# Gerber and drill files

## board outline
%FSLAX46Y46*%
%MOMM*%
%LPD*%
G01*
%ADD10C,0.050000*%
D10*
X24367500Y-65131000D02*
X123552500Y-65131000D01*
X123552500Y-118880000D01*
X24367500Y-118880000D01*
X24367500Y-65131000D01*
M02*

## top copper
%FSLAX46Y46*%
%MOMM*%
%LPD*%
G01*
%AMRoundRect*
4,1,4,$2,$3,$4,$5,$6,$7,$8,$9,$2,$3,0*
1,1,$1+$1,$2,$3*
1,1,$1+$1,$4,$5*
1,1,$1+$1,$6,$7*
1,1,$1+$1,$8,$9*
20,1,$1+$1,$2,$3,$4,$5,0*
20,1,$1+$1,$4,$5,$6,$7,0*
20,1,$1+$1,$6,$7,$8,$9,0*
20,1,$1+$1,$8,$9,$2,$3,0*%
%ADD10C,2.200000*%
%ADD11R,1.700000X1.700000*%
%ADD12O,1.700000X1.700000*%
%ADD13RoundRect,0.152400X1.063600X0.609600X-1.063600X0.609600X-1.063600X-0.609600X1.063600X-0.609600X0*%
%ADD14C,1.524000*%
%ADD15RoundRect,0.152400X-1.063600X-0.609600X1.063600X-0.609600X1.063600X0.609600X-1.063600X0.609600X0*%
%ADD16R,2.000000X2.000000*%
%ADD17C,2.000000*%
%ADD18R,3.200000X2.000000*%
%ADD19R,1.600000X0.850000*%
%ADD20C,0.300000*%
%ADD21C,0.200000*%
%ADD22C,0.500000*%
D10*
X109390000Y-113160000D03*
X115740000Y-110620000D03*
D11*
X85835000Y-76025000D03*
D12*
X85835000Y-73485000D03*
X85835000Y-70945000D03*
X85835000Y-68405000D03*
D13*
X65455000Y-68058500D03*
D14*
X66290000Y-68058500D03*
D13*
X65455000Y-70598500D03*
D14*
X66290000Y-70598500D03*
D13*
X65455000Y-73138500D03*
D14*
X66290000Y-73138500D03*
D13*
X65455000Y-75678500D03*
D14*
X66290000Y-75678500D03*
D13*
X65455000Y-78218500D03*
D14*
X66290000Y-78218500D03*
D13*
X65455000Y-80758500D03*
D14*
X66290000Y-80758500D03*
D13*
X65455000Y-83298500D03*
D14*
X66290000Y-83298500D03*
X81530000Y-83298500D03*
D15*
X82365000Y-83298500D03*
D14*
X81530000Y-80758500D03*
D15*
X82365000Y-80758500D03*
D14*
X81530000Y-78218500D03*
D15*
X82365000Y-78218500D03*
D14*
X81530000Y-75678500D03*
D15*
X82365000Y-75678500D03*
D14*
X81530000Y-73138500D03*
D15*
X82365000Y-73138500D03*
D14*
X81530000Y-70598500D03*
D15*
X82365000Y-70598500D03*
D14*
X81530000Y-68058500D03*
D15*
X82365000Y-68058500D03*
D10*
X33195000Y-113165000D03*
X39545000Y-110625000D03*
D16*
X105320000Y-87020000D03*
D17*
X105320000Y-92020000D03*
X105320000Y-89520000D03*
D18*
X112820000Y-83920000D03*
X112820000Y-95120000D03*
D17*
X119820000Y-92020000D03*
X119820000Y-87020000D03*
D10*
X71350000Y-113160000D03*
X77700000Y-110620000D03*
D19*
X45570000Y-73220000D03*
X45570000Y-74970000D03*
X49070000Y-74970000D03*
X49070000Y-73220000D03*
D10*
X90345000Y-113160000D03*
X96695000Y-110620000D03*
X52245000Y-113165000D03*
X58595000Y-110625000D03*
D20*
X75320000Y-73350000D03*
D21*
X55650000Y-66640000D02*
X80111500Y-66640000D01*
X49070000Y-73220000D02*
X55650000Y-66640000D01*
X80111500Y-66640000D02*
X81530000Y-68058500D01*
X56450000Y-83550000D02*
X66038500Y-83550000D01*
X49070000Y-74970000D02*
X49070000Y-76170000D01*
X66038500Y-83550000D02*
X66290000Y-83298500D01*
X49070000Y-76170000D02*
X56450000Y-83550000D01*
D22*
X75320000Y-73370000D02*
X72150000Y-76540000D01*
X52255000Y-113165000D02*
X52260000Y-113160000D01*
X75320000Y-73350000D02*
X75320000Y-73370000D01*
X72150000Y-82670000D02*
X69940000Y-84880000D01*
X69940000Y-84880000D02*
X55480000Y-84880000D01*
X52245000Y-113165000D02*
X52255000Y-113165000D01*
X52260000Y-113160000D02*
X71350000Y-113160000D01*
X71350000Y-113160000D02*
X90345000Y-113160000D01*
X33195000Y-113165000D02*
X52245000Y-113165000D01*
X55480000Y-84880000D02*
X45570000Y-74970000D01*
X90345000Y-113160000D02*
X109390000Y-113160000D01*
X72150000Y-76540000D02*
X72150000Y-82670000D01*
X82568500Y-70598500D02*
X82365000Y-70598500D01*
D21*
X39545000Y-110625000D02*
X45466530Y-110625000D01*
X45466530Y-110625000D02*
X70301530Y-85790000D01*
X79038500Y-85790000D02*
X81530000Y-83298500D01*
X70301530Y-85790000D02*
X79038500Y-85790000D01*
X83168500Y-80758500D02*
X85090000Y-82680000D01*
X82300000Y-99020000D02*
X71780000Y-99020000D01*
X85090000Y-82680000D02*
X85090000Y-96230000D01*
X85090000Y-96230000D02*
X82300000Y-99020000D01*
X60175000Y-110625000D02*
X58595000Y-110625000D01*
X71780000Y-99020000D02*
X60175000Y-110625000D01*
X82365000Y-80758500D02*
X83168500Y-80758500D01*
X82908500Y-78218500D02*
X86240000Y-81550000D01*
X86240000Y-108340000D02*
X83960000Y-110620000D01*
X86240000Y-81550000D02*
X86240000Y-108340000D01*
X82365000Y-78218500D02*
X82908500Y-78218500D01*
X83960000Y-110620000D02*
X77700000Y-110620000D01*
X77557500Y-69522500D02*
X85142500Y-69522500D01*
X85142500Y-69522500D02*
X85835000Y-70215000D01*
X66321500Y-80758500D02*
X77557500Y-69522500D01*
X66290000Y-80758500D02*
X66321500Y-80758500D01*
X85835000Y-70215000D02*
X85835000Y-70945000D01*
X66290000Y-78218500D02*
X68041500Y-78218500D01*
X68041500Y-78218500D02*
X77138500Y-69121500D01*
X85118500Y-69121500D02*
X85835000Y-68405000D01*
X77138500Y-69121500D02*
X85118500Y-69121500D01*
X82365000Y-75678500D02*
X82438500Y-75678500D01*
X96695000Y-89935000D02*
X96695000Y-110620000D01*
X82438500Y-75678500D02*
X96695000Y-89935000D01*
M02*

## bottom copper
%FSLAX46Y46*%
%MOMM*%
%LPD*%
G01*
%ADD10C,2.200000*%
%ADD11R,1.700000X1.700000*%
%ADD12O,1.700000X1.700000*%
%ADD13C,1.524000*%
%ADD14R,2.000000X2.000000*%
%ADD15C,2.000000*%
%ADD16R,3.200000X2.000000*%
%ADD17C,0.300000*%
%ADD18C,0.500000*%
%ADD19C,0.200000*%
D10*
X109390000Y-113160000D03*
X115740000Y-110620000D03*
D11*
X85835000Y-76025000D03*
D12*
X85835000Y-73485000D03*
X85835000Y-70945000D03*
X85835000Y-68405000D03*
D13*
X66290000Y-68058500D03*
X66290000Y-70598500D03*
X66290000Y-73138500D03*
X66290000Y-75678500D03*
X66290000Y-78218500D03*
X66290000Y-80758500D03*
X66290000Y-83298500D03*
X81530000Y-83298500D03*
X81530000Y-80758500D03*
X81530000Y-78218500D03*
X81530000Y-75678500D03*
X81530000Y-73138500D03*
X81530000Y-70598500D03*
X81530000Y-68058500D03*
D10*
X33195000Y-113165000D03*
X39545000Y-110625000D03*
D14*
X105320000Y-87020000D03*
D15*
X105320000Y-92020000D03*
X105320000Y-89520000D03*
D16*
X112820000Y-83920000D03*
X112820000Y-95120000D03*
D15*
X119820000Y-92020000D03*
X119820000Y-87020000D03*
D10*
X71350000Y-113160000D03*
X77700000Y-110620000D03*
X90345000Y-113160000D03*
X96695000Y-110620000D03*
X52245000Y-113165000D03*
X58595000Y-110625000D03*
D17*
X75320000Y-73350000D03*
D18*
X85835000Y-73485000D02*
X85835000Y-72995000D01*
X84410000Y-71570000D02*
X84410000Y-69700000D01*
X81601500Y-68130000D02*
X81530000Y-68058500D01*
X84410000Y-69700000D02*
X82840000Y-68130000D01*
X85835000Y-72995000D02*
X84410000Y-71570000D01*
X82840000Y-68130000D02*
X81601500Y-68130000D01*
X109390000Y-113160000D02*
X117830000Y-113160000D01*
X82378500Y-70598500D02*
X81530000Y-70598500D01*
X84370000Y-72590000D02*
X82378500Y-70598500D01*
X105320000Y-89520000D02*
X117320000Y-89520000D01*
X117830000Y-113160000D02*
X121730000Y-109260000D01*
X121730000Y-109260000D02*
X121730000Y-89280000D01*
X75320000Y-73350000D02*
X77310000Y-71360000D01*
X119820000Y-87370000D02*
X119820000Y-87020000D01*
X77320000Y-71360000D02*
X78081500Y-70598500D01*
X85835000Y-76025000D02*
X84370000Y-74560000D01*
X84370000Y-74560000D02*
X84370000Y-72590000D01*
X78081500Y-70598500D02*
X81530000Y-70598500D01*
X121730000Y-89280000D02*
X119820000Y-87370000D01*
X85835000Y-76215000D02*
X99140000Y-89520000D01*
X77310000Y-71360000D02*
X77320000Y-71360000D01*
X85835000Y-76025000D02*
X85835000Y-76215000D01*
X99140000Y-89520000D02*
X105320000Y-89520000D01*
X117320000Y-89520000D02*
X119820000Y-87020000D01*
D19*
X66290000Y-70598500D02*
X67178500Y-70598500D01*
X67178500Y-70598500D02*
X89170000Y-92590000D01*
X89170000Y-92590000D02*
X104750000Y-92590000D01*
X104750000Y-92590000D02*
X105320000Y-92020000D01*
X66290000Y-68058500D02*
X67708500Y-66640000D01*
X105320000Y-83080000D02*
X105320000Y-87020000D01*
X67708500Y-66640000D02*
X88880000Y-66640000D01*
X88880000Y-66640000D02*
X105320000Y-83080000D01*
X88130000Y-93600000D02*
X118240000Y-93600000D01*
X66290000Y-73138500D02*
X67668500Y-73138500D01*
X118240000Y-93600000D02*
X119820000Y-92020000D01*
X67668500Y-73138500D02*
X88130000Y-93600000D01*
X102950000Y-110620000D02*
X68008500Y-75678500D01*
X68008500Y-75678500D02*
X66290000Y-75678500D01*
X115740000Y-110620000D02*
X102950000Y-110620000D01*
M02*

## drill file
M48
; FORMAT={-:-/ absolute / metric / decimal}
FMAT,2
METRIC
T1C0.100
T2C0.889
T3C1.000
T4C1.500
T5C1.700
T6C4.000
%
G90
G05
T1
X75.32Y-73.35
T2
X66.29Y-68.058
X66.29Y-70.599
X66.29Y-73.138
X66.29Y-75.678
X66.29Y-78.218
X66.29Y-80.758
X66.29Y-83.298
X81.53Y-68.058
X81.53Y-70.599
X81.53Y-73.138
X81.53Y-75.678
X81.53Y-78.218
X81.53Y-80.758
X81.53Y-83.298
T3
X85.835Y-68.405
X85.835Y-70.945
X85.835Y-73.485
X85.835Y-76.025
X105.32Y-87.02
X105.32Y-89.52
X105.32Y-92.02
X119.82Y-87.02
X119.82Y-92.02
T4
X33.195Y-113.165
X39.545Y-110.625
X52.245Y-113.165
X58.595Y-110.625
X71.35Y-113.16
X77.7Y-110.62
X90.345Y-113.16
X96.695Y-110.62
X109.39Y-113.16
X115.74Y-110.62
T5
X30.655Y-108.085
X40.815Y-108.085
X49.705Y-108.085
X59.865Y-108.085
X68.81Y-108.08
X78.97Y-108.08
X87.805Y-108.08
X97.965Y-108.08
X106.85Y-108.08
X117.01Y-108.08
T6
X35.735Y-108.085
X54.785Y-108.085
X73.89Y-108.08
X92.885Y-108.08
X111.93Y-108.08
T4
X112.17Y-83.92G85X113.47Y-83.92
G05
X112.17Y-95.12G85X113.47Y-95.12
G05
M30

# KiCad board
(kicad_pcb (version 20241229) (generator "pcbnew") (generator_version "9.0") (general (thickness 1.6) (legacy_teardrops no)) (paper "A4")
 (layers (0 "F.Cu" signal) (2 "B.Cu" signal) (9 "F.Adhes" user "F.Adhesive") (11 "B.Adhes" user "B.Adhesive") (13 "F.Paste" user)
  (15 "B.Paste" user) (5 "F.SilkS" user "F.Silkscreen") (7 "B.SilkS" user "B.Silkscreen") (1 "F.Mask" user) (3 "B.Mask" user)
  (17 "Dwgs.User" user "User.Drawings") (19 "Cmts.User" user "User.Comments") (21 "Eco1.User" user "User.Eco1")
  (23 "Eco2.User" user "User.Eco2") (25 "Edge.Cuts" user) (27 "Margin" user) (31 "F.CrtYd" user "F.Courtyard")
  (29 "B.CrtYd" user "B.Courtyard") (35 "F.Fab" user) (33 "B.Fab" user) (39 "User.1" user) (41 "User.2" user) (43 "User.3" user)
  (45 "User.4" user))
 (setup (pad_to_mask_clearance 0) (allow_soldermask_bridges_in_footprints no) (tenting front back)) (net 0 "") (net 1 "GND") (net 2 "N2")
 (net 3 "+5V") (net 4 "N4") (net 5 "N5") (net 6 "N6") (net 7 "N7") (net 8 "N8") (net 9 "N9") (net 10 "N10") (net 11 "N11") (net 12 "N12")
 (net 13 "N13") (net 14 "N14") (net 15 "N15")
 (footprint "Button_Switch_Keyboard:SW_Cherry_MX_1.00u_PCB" (layer "F.Cu") (at 109.39 113.16 180)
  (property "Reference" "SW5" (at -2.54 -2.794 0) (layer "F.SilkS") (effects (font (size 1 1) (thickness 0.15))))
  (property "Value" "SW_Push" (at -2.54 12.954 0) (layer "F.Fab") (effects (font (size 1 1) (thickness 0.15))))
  (pad "" np_thru_hole circle (at -7.62 5.08 180) (size 1.7 1.7) (drill 1.7) (layers "*.Cu" "*.Mask"))
  (pad "" np_thru_hole circle (at -2.54 5.08 180) (size 4 4) (drill 4) (layers "*.Cu" "*.Mask"))
  (pad "" np_thru_hole circle (at 2.54 5.08 180) (size 1.7 1.7) (drill 1.7) (layers "*.Cu" "*.Mask"))
  (pad "1" thru_hole circle (at 0 0 180) (size 2.2 2.2) (drill 1.5) (layers "*.Cu" "*.Mask") (remove_unused_layers no) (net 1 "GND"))
  (pad "2" thru_hole circle (at -6.35 2.54 180) (size 2.2 2.2) (drill 1.5) (layers "*.Cu" "*.Mask") (remove_unused_layers no) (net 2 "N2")))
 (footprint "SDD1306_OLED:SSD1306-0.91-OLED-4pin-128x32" (layer "F.Cu") (at 122.335 78.215 180)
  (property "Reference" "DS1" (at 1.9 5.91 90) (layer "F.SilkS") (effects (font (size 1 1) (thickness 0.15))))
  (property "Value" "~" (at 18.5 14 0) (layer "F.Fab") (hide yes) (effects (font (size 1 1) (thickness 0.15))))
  (pad "1" thru_hole rect (at 36.5 2.19 180) (size 1.7 1.7) (drill 1) (layers "*.Cu" "*.Mask") (remove_unused_layers no) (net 1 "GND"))
  (pad "2" thru_hole oval (at 36.5 4.73 180) (size 1.7 1.7) (drill 1) (layers "*.Cu" "*.Mask") (remove_unused_layers no) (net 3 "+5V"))
  (pad "3" thru_hole oval (at 36.5 7.27 180) (size 1.7 1.7) (drill 1) (layers "*.Cu" "*.Mask") (remove_unused_layers no) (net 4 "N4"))
  (pad "4" thru_hole oval (at 36.5 9.81 180) (size 1.7 1.7) (drill 1) (layers "*.Cu" "*.Mask") (remove_unused_layers no) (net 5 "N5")))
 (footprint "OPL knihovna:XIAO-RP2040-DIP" (layer "F.Cu") (at 73.91 75.6785)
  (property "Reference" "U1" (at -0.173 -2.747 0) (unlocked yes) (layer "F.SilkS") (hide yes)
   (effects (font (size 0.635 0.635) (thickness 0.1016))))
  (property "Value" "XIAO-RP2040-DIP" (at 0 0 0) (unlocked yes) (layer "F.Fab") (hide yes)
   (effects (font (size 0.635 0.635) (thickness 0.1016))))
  (pad "1" smd roundrect (at -8.455 -7.62 180) (size 2.432 1.524) (layers "F.Cu" "F.Mask") (roundrect_rratio 0.1) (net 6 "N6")
   (thermal_bridge_angle 45))
  (pad "1" thru_hole circle (at -7.62 -7.62 180) (size 1.524 1.524) (drill 0.889) (layers "*.Cu" "*.Mask") (remove_unused_layers no)
   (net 6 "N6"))
  (pad "2" smd roundrect (at -8.455 -5.08 180) (size 2.432 1.524) (layers "F.Cu" "F.Mask") (roundrect_rratio 0.1) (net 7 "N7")
   (thermal_bridge_angle 45))
  (pad "2" thru_hole circle (at -7.62 -5.08 180) (size 1.524 1.524) (drill 0.889) (layers "*.Cu" "*.Mask") (remove_unused_layers no)
   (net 7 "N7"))
  (pad "3" smd roundrect (at -8.455 -2.54 180) (size 2.432 1.524) (layers "F.Cu" "F.Mask") (roundrect_rratio 0.1) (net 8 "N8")
   (thermal_bridge_angle 45))
  (pad "3" thru_hole circle (at -7.62 -2.54 180) (size 1.524 1.524) (drill 0.889) (layers "*.Cu" "*.Mask") (remove_unused_layers no)
   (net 8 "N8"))
  (pad "4" smd roundrect (at -8.455 0 180) (size 2.432 1.524) (layers "F.Cu" "F.Mask") (roundrect_rratio 0.1) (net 2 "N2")
   (thermal_bridge_angle 45))
  (pad "4" thru_hole circle (at -7.62 0 180) (size 1.524 1.524) (drill 0.889) (layers "*.Cu" "*.Mask") (remove_unused_layers no)
   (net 2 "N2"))
  (pad "5" smd roundrect (at -8.455 2.54 180) (size 2.432 1.524) (layers "F.Cu" "F.Mask") (roundrect_rratio 0.1) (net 5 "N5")
   (thermal_bridge_angle 45))
  (pad "5" thru_hole circle (at -7.62 2.54 180) (size 1.524 1.524) (drill 0.889) (layers "*.Cu" "*.Mask") (remove_unused_layers no)
   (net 5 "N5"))
  (pad "6" smd roundrect (at -8.455 5.08 180) (size 2.432 1.524) (layers "F.Cu" "F.Mask") (roundrect_rratio 0.1) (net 4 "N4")
   (thermal_bridge_angle 45))
  (pad "6" thru_hole circle (at -7.62 5.08 180) (size 1.524 1.524) (drill 0.889) (layers "*.Cu" "*.Mask") (remove_unused_layers no)
   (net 4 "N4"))
  (pad "7" smd roundrect (at -8.455 7.62 180) (size 2.432 1.524) (layers "F.Cu" "F.Mask") (roundrect_rratio 0.1) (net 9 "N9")
   (thermal_bridge_angle 45))
  (pad "7" thru_hole circle (at -7.62 7.62 180) (size 1.524 1.524) (drill 0.889) (layers "*.Cu" "*.Mask") (remove_unused_layers no)
   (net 9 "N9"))
  (pad "8" thru_hole circle (at 7.62 7.62) (size 1.524 1.524) (drill 0.889) (layers "*.Cu" "*.Mask") (remove_unused_layers no)
   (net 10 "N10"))
  (pad "8" smd roundrect (at 8.455 7.62) (size 2.432 1.524) (layers "F.Cu" "F.Mask") (roundrect_rratio 0.1) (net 10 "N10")
   (thermal_bridge_angle 45))
  (pad "9" thru_hole circle (at 7.62 5.08) (size 1.524 1.524) (drill 0.889) (layers "*.Cu" "*.Mask") (remove_unused_layers no)
   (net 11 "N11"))
  (pad "9" smd roundrect (at 8.455 5.08) (size 2.432 1.524) (layers "F.Cu" "F.Mask") (roundrect_rratio 0.1) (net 11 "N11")
   (thermal_bridge_angle 45))
  (pad "10" thru_hole circle (at 7.62 2.54) (size 1.524 1.524) (drill 0.889) (layers "*.Cu" "*.Mask") (remove_unused_layers no)
   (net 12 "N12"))
  (pad "10" smd roundrect (at 8.455 2.54) (size 2.432 1.524) (layers "F.Cu" "F.Mask") (roundrect_rratio 0.1) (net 12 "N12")
   (thermal_bridge_angle 45))
  (pad "11" thru_hole circle (at 7.62 0) (size 1.524 1.524) (drill 0.889) (layers "*.Cu" "*.Mask") (remove_unused_layers no) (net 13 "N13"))
  (pad "11" smd roundrect (at 8.455 0) (size 2.432 1.524) (layers "F.Cu" "F.Mask") (roundrect_rratio 0.1) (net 13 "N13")
   (thermal_bridge_angle 45))
  (pad "12" thru_hole circle (at 7.62 -2.54) (size 1.524 1.524) (drill 0.889) (layers "*.Cu" "*.Mask") (remove_unused_layers no)
   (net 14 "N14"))
  (pad "12" smd roundrect (at 8.455 -2.54) (size 2.432 1.524) (layers "F.Cu" "F.Mask") (roundrect_rratio 0.1) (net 14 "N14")
   (thermal_bridge_angle 45))
  (pad "13" thru_hole circle (at 7.62 -5.08) (size 1.524 1.524) (drill 0.889) (layers "*.Cu" "*.Mask") (remove_unused_layers no)
   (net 1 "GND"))
  (pad "13" smd roundrect (at 8.455 -5.08) (size 2.432 1.524) (layers "F.Cu" "F.Mask") (roundrect_rratio 0.1) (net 1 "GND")
   (thermal_bridge_angle 45))
  (pad "14" thru_hole circle (at 7.62 -7.62) (size 1.524 1.524) (drill 0.889) (layers "*.Cu" "*.Mask") (remove_unused_layers no)
   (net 3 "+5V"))
  (pad "14" smd roundrect (at 8.455 -7.62) (size 2.432 1.524) (layers "F.Cu" "F.Mask") (roundrect_rratio 0.1) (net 3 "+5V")
   (thermal_bridge_angle 45)))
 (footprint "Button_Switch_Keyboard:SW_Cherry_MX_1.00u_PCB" (layer "F.Cu") (at 33.195 113.165 180)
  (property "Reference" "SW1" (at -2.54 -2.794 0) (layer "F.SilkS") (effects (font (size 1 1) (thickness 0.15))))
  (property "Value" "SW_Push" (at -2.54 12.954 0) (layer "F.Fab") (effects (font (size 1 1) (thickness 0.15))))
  (pad "" np_thru_hole circle (at -7.62 5.08 180) (size 1.7 1.7) (drill 1.7) (layers "*.Cu" "*.Mask"))
  (pad "" np_thru_hole circle (at -2.54 5.08 180) (size 4 4) (drill 4) (layers "*.Cu" "*.Mask"))
  (pad "" np_thru_hole circle (at 2.54 5.08 180) (size 1.7 1.7) (drill 1.7) (layers "*.Cu" "*.Mask"))
  (pad "1" thru_hole circle (at 0 0 180) (size 2.2 2.2) (drill 1.5) (layers "*.Cu" "*.Mask") (remove_unused_layers no) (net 1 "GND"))
  (pad "2" thru_hole circle (at -6.35 2.54 180) (size 2.2 2.2) (drill 1.5) (layers "*.Cu" "*.Mask") (remove_unused_layers no) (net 10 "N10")))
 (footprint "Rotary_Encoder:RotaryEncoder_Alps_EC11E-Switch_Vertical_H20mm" (layer "F.Cu") (at 105.32 87.02)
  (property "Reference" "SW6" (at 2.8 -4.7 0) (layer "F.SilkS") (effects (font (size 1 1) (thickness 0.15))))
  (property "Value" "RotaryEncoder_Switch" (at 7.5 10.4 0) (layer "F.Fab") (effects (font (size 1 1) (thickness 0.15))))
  (pad "A" thru_hole rect (at 0 0) (size 2 2) (drill 1) (layers "*.Cu" "*.Mask") (remove_unused_layers no) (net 6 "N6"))
  (pad "B" thru_hole circle (at 0 5) (size 2 2) (drill 1) (layers "*.Cu" "*.Mask") (remove_unused_layers no) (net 7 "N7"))
  (pad "C" thru_hole circle (at 0 2.5) (size 2 2) (drill 1) (layers "*.Cu" "*.Mask") (remove_unused_layers no) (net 1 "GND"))
  (pad "MP" thru_hole rect (at 7.5 -3.1) (size 3.2 2) (drill oval 2.8 1.5) (layers "*.Cu" "*.Mask") (remove_unused_layers no))
  (pad "MP" thru_hole rect (at 7.5 8.1) (size 3.2 2) (drill oval 2.8 1.5) (layers "*.Cu" "*.Mask") (remove_unused_layers no))
  (pad "S1" thru_hole circle (at 14.5 5) (size 2 2) (drill 1) (layers "*.Cu" "*.Mask") (remove_unused_layers no) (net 8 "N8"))
  (pad "S2" thru_hole circle (at 14.5 0) (size 2 2) (drill 1) (layers "*.Cu" "*.Mask") (remove_unused_layers no) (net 1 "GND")))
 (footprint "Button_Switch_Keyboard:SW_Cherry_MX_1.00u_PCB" (layer "F.Cu") (at 71.35 113.16 180)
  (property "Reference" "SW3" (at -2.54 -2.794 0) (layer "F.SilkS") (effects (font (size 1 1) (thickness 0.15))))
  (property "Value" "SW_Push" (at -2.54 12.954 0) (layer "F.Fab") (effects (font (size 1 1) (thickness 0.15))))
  (pad "" np_thru_hole circle (at -7.62 5.08 180) (size 1.7 1.7) (drill 1.7) (layers "*.Cu" "*.Mask"))
  (pad "" np_thru_hole circle (at -2.54 5.08 180) (size 4 4) (drill 4) (layers "*.Cu" "*.Mask"))
  (pad "" np_thru_hole circle (at 2.54 5.08 180) (size 1.7 1.7) (drill 1.7) (layers "*.Cu" "*.Mask"))
  (pad "1" thru_hole circle (at 0 0 180) (size 2.2 2.2) (drill 1.5) (layers "*.Cu" "*.Mask") (remove_unused_layers no) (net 1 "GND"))
  (pad "2" thru_hole circle (at -6.35 2.54 180) (size 2.2 2.2) (drill 1.5) (layers "*.Cu" "*.Mask") (remove_unused_layers no) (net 12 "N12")))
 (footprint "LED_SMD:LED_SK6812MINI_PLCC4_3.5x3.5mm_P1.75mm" (layer "F.Cu") (at 47.32 74.095)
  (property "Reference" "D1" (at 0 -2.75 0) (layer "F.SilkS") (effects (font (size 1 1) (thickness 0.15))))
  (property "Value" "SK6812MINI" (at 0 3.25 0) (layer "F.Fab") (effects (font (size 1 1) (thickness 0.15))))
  (pad "1" smd rect (at -1.75 -0.875) (size 1.6 0.85) (layers "F.Cu" "F.Mask" "F.Paste") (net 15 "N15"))
  (pad "2" smd rect (at -1.75 0.875) (size 1.6 0.85) (layers "F.Cu" "F.Mask" "F.Paste") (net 1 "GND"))
  (pad "3" smd rect (at 1.75 0.875) (size 1.6 0.85) (layers "F.Cu" "F.Mask" "F.Paste") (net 9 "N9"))
  (pad "4" smd rect (at 1.75 -0.875) (size 1.6 0.85) (layers "F.Cu" "F.Mask" "F.Paste") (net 3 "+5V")))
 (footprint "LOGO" (layer "F.Cu") (at 44.39 80.29)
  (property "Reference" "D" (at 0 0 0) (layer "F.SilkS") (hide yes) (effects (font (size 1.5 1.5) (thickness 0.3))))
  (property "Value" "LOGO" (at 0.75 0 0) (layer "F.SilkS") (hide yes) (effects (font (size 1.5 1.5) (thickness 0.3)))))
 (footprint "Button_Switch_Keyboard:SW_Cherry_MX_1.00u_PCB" (layer "F.Cu") (at 90.345 113.16 180)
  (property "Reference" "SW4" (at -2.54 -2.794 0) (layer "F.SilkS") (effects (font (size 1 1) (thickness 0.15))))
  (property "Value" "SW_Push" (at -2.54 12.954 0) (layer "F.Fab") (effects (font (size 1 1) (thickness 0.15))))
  (pad "" np_thru_hole circle (at -7.62 5.08 180) (size 1.7 1.7) (drill 1.7) (layers "*.Cu" "*.Mask"))
  (pad "" np_thru_hole circle (at -2.54 5.08 180) (size 4 4) (drill 4) (layers "*.Cu" "*.Mask"))
  (pad "" np_thru_hole circle (at 2.54 5.08 180) (size 1.7 1.7) (drill 1.7) (layers "*.Cu" "*.Mask"))
  (pad "1" thru_hole circle (at 0 0 180) (size 2.2 2.2) (drill 1.5) (layers "*.Cu" "*.Mask") (remove_unused_layers no) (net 1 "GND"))
  (pad "2" thru_hole circle (at -6.35 2.54 180) (size 2.2 2.2) (drill 1.5) (layers "*.Cu" "*.Mask") (remove_unused_layers no) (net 13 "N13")))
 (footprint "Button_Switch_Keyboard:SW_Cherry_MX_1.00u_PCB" (layer "F.Cu") (at 52.245 113.165 180)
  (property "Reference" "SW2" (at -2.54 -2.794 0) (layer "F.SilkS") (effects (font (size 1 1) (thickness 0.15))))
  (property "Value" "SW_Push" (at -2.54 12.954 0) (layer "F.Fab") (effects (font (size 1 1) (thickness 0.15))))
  (pad "" np_thru_hole circle (at -7.62 5.08 180) (size 1.7 1.7) (drill 1.7) (layers "*.Cu" "*.Mask"))
  (pad "" np_thru_hole circle (at -2.54 5.08 180) (size 4 4) (drill 4) (layers "*.Cu" "*.Mask"))
  (pad "" np_thru_hole circle (at 2.54 5.08 180) (size 1.7 1.7) (drill 1.7) (layers "*.Cu" "*.Mask"))
  (pad "1" thru_hole circle (at 0 0 180) (size 2.2 2.2) (drill 1.5) (layers "*.Cu" "*.Mask") (remove_unused_layers no) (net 1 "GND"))
  (pad "2" thru_hole circle (at -6.35 2.54 180) (size 2.2 2.2) (drill 1.5) (layers "*.Cu" "*.Mask") (remove_unused_layers no) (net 11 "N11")))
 (gr_rect (start 24.3675 65.131) (end 123.5525 118.88) (stroke (width 0.05) (type default)) (fill no) (layer "Edge.Cuts"))
 (segment (start 55.65 66.64) (end 80.1115 66.64) (width 0.2) (layer "F.Cu") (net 3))
 (segment (start 49.07 73.22) (end 55.65 66.64) (width 0.2) (layer "F.Cu") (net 3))
 (segment (start 80.1115 66.64) (end 81.53 68.0585) (width 0.2) (layer "F.Cu") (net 3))
 (segment (start 85.835 73.485) (end 85.835 72.995) (width 0.5) (layer "B.Cu") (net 3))
 (segment (start 84.41 71.57) (end 84.41 69.7) (width 0.5) (layer "B.Cu") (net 3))
 (segment (start 81.6015 68.13) (end 81.53 68.0585) (width 0.5) (layer "B.Cu") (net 3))
 (segment (start 84.41 69.7) (end 82.84 68.13) (width 0.5) (layer "B.Cu") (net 3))
 (segment (start 85.835 72.995) (end 84.41 71.57) (width 0.5) (layer "B.Cu") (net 3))
 (segment (start 82.84 68.13) (end 81.6015 68.13) (width 0.5) (layer "B.Cu") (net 3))
 (segment (start 56.45 83.55) (end 66.0385 83.55) (width 0.2) (layer "F.Cu") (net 9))
 (segment (start 49.07 74.97) (end 49.07 76.17) (width 0.2) (layer "F.Cu") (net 9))
 (segment (start 66.0385 83.55) (end 66.29 83.2985) (width 0.2) (layer "F.Cu") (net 9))
 (segment (start 49.07 76.17) (end 56.45 83.55) (width 0.2) (layer "F.Cu") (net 9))
 (segment (start 75.32 73.37) (end 72.15 76.54) (width 0.5) (layer "F.Cu") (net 1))
 (segment (start 52.255 113.165) (end 52.26 113.16) (width 0.5) (layer "F.Cu") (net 1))
 (segment (start 75.32 73.35) (end 75.32 73.37) (width 0.5) (layer "F.Cu") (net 1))
 (segment (start 72.15 82.67) (end 69.94 84.88) (width 0.5) (layer "F.Cu") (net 1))
 (segment (start 69.94 84.88) (end 55.48 84.88) (width 0.5) (layer "F.Cu") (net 1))
 (segment (start 52.245 113.165) (end 52.255 113.165) (width 0.5) (layer "F.Cu") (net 1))
 (segment (start 52.26 113.16) (end 71.35 113.16) (width 0.5) (layer "F.Cu") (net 1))
 (segment (start 71.35 113.16) (end 90.345 113.16) (width 0.5) (layer "F.Cu") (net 1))
 (segment (start 33.195 113.165) (end 52.245 113.165) (width 0.5) (layer "F.Cu") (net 1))
 (segment (start 55.48 84.88) (end 45.57 74.97) (width 0.5) (layer "F.Cu") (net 1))
 (segment (start 90.345 113.16) (end 109.39 113.16) (width 0.5) (layer "F.Cu") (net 1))
 (segment (start 72.15 76.54) (end 72.15 82.67) (width 0.5) (layer "F.Cu") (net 1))
 (segment (start 82.5685 70.5985) (end 82.365 70.5985) (width 0.5) (layer "F.Cu") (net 1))
 (via micro (at 75.32 73.35) (size 0.3) (drill 0.1) (layers "F.Cu" "B.Cu") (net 1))
 (segment (start 109.39 113.16) (end 117.83 113.16) (width 0.5) (layer "B.Cu") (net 1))
 (segment (start 82.3785 70.5985) (end 81.53 70.5985) (width 0.5) (layer "B.Cu") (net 1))
 (segment (start 84.37 72.59) (end 82.3785 70.5985) (width 0.5) (layer "B.Cu") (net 1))
 (segment (start 105.32 89.52) (end 117.32 89.52) (width 0.5) (layer "B.Cu") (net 1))
 (segment (start 117.83 113.16) (end 121.73 109.26) (width 0.5) (layer "B.Cu") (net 1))
 (segment (start 121.73 109.26) (end 121.73 89.28) (width 0.5) (layer "B.Cu") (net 1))
 (segment (start 75.32 73.35) (end 77.31 71.36) (width 0.5) (layer "B.Cu") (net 1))
 (segment (start 119.82 87.37) (end 119.82 87.02) (width 0.5) (layer "B.Cu") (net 1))
 (segment (start 77.32 71.36) (end 78.0815 70.5985) (width 0.5) (layer "B.Cu") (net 1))
 (segment (start 85.835 76.025) (end 84.37 74.56) (width 0.5) (layer "B.Cu") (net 1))
 (segment (start 84.37 74.56) (end 84.37 72.59) (width 0.5) (layer "B.Cu") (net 1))
 (segment (start 78.0815 70.5985) (end 81.53 70.5985) (width 0.5) (layer "B.Cu") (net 1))
 (segment (start 121.73 89.28) (end 119.82 87.37) (width 0.5) (layer "B.Cu") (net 1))
 (segment (start 85.835 76.215) (end 99.14 89.52) (width 0.5) (layer "B.Cu") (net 1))
 (segment (start 77.31 71.36) (end 77.32 71.36) (width 0.5) (layer "B.Cu") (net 1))
 (segment (start 85.835 76.025) (end 85.835 76.215) (width 0.5) (layer "B.Cu") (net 1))
 (segment (start 99.14 89.52) (end 105.32 89.52) (width 0.5) (layer "B.Cu") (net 1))
 (segment (start 117.32 89.52) (end 119.82 87.02) (width 0.5) (layer "B.Cu") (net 1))
 (segment (start 39.545 110.625) (end 45.46653 110.625) (width 0.2) (layer "F.Cu") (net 10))
 (segment (start 45.46653 110.625) (end 70.30153 85.79) (width 0.2) (layer "F.Cu") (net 10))
 (segment (start 79.0385 85.79) (end 81.53 83.2985) (width 0.2) (layer "F.Cu") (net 10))
 (segment (start 70.30153 85.79) (end 79.0385 85.79) (width 0.2) (layer "F.Cu") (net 10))
 (segment (start 83.1685 80.7585) (end 85.09 82.68) (width 0.2) (layer "F.Cu") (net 11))
 (segment (start 82.3 99.02) (end 71.78 99.02) (width 0.2) (layer "F.Cu") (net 11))
 (segment (start 85.09 82.68) (end 85.09 96.23) (width 0.2) (layer "F.Cu") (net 11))
 (segment (start 85.09 96.23) (end 82.3 99.02) (width 0.2) (layer "F.Cu") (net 11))
 (segment (start 60.175 110.625) (end 58.595 110.625) (width 0.2) (layer "F.Cu") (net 11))
 (segment (start 71.78 99.02) (end 60.175 110.625) (width 0.2) (layer "F.Cu") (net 11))
 (segment (start 82.365 80.7585) (end 83.1685 80.7585) (width 0.2) (layer "F.Cu") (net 11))
 (segment (start 82.9085 78.2185) (end 86.24 81.55) (width 0.2) (layer "F.Cu") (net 12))
 (segment (start 86.24 108.34) (end 83.96 110.62) (width 0.2) (layer "F.Cu") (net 12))
 (segment (start 86.24 81.55) (end 86.24 108.34) (width 0.2) (layer "F.Cu") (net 12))
 (segment (start 82.365 78.2185) (end 82.9085 78.2185) (width 0.2) (layer "F.Cu") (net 12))
 (segment (start 83.96 110.62) (end 77.7 110.62) (width 0.2) (layer "F.Cu") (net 12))
 (segment (start 77.5575 69.5225) (end 85.1425 69.5225) (width 0.2) (layer "F.Cu") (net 4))
 (segment (start 85.1425 69.5225) (end 85.835 70.215) (width 0.2) (layer "F.Cu") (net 4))
 (segment (start 66.3215 80.7585) (end 77.5575 69.5225) (width 0.2) (layer "F.Cu") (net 4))
 (segment (start 66.29 80.7585) (end 66.3215 80.7585) (width 0.2) (layer "F.Cu") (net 4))
 (segment (start 85.835 70.215) (end 85.835 70.945) (width 0.2) (layer "F.Cu") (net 4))
 (segment (start 66.29 78.2185) (end 68.0415 78.2185) (width 0.2) (layer "F.Cu") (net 5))
 (segment (start 68.0415 78.2185) (end 77.1385 69.1215) (width 0.2) (layer "F.Cu") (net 5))
 (segment (start 85.1185 69.1215) (end 85.835 68.405) (width 0.2) (layer "F.Cu") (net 5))
 (segment (start 77.1385 69.1215) (end 85.1185 69.1215) (width 0.2) (layer "F.Cu") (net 5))
 (segment (start 66.29 70.5985) (end 67.1785 70.5985) (width 0.2) (layer "B.Cu") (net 7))
 (segment (start 67.1785 70.5985) (end 89.17 92.59) (width 0.2) (layer "B.Cu") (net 7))
 (segment (start 89.17 92.59) (end 104.75 92.59) (width 0.2) (layer "B.Cu") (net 7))
 (segment (start 104.75 92.59) (end 105.32 92.02) (width 0.2) (layer "B.Cu") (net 7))
 (segment (start 66.29 68.0585) (end 67.7085 66.64) (width 0.2) (layer "B.Cu") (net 6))
 (segment (start 105.32 83.08) (end 105.32 87.02) (width 0.2) (layer "B.Cu") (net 6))
 (segment (start 67.7085 66.64) (end 88.88 66.64) (width 0.2) (layer "B.Cu") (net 6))
 (segment (start 88.88 66.64) (end 105.32 83.08) (width 0.2) (layer "B.Cu") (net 6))
 (segment (start 88.13 93.6) (end 118.24 93.6) (width 0.2) (layer "B.Cu") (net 8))
 (segment (start 66.29 73.1385) (end 67.6685 73.1385) (width 0.2) (layer "B.Cu") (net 8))
 (segment (start 118.24 93.6) (end 119.82 92.02) (width 0.2) (layer "B.Cu") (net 8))
 (segment (start 67.6685 73.1385) (end 88.13 93.6) (width 0.2) (layer "B.Cu") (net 8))
 (segment (start 102.95 110.62) (end 68.0085 75.6785) (width 0.2) (layer "B.Cu") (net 2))
 (segment (start 68.0085 75.6785) (end 66.29 75.6785) (width 0.2) (layer "B.Cu") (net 2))
 (segment (start 115.74 110.62) (end 102.95 110.62) (width 0.2) (layer "B.Cu") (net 2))
 (segment (start 82.365 75.6785) (end 82.4385 75.6785) (width 0.2) (layer "F.Cu") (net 13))
 (segment (start 96.695 89.935) (end 96.695 110.62) (width 0.2) (layer "F.Cu") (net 13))
 (segment (start 82.4385 75.6785) (end 96.695 89.935) (width 0.2) (layer "F.Cu") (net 13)))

